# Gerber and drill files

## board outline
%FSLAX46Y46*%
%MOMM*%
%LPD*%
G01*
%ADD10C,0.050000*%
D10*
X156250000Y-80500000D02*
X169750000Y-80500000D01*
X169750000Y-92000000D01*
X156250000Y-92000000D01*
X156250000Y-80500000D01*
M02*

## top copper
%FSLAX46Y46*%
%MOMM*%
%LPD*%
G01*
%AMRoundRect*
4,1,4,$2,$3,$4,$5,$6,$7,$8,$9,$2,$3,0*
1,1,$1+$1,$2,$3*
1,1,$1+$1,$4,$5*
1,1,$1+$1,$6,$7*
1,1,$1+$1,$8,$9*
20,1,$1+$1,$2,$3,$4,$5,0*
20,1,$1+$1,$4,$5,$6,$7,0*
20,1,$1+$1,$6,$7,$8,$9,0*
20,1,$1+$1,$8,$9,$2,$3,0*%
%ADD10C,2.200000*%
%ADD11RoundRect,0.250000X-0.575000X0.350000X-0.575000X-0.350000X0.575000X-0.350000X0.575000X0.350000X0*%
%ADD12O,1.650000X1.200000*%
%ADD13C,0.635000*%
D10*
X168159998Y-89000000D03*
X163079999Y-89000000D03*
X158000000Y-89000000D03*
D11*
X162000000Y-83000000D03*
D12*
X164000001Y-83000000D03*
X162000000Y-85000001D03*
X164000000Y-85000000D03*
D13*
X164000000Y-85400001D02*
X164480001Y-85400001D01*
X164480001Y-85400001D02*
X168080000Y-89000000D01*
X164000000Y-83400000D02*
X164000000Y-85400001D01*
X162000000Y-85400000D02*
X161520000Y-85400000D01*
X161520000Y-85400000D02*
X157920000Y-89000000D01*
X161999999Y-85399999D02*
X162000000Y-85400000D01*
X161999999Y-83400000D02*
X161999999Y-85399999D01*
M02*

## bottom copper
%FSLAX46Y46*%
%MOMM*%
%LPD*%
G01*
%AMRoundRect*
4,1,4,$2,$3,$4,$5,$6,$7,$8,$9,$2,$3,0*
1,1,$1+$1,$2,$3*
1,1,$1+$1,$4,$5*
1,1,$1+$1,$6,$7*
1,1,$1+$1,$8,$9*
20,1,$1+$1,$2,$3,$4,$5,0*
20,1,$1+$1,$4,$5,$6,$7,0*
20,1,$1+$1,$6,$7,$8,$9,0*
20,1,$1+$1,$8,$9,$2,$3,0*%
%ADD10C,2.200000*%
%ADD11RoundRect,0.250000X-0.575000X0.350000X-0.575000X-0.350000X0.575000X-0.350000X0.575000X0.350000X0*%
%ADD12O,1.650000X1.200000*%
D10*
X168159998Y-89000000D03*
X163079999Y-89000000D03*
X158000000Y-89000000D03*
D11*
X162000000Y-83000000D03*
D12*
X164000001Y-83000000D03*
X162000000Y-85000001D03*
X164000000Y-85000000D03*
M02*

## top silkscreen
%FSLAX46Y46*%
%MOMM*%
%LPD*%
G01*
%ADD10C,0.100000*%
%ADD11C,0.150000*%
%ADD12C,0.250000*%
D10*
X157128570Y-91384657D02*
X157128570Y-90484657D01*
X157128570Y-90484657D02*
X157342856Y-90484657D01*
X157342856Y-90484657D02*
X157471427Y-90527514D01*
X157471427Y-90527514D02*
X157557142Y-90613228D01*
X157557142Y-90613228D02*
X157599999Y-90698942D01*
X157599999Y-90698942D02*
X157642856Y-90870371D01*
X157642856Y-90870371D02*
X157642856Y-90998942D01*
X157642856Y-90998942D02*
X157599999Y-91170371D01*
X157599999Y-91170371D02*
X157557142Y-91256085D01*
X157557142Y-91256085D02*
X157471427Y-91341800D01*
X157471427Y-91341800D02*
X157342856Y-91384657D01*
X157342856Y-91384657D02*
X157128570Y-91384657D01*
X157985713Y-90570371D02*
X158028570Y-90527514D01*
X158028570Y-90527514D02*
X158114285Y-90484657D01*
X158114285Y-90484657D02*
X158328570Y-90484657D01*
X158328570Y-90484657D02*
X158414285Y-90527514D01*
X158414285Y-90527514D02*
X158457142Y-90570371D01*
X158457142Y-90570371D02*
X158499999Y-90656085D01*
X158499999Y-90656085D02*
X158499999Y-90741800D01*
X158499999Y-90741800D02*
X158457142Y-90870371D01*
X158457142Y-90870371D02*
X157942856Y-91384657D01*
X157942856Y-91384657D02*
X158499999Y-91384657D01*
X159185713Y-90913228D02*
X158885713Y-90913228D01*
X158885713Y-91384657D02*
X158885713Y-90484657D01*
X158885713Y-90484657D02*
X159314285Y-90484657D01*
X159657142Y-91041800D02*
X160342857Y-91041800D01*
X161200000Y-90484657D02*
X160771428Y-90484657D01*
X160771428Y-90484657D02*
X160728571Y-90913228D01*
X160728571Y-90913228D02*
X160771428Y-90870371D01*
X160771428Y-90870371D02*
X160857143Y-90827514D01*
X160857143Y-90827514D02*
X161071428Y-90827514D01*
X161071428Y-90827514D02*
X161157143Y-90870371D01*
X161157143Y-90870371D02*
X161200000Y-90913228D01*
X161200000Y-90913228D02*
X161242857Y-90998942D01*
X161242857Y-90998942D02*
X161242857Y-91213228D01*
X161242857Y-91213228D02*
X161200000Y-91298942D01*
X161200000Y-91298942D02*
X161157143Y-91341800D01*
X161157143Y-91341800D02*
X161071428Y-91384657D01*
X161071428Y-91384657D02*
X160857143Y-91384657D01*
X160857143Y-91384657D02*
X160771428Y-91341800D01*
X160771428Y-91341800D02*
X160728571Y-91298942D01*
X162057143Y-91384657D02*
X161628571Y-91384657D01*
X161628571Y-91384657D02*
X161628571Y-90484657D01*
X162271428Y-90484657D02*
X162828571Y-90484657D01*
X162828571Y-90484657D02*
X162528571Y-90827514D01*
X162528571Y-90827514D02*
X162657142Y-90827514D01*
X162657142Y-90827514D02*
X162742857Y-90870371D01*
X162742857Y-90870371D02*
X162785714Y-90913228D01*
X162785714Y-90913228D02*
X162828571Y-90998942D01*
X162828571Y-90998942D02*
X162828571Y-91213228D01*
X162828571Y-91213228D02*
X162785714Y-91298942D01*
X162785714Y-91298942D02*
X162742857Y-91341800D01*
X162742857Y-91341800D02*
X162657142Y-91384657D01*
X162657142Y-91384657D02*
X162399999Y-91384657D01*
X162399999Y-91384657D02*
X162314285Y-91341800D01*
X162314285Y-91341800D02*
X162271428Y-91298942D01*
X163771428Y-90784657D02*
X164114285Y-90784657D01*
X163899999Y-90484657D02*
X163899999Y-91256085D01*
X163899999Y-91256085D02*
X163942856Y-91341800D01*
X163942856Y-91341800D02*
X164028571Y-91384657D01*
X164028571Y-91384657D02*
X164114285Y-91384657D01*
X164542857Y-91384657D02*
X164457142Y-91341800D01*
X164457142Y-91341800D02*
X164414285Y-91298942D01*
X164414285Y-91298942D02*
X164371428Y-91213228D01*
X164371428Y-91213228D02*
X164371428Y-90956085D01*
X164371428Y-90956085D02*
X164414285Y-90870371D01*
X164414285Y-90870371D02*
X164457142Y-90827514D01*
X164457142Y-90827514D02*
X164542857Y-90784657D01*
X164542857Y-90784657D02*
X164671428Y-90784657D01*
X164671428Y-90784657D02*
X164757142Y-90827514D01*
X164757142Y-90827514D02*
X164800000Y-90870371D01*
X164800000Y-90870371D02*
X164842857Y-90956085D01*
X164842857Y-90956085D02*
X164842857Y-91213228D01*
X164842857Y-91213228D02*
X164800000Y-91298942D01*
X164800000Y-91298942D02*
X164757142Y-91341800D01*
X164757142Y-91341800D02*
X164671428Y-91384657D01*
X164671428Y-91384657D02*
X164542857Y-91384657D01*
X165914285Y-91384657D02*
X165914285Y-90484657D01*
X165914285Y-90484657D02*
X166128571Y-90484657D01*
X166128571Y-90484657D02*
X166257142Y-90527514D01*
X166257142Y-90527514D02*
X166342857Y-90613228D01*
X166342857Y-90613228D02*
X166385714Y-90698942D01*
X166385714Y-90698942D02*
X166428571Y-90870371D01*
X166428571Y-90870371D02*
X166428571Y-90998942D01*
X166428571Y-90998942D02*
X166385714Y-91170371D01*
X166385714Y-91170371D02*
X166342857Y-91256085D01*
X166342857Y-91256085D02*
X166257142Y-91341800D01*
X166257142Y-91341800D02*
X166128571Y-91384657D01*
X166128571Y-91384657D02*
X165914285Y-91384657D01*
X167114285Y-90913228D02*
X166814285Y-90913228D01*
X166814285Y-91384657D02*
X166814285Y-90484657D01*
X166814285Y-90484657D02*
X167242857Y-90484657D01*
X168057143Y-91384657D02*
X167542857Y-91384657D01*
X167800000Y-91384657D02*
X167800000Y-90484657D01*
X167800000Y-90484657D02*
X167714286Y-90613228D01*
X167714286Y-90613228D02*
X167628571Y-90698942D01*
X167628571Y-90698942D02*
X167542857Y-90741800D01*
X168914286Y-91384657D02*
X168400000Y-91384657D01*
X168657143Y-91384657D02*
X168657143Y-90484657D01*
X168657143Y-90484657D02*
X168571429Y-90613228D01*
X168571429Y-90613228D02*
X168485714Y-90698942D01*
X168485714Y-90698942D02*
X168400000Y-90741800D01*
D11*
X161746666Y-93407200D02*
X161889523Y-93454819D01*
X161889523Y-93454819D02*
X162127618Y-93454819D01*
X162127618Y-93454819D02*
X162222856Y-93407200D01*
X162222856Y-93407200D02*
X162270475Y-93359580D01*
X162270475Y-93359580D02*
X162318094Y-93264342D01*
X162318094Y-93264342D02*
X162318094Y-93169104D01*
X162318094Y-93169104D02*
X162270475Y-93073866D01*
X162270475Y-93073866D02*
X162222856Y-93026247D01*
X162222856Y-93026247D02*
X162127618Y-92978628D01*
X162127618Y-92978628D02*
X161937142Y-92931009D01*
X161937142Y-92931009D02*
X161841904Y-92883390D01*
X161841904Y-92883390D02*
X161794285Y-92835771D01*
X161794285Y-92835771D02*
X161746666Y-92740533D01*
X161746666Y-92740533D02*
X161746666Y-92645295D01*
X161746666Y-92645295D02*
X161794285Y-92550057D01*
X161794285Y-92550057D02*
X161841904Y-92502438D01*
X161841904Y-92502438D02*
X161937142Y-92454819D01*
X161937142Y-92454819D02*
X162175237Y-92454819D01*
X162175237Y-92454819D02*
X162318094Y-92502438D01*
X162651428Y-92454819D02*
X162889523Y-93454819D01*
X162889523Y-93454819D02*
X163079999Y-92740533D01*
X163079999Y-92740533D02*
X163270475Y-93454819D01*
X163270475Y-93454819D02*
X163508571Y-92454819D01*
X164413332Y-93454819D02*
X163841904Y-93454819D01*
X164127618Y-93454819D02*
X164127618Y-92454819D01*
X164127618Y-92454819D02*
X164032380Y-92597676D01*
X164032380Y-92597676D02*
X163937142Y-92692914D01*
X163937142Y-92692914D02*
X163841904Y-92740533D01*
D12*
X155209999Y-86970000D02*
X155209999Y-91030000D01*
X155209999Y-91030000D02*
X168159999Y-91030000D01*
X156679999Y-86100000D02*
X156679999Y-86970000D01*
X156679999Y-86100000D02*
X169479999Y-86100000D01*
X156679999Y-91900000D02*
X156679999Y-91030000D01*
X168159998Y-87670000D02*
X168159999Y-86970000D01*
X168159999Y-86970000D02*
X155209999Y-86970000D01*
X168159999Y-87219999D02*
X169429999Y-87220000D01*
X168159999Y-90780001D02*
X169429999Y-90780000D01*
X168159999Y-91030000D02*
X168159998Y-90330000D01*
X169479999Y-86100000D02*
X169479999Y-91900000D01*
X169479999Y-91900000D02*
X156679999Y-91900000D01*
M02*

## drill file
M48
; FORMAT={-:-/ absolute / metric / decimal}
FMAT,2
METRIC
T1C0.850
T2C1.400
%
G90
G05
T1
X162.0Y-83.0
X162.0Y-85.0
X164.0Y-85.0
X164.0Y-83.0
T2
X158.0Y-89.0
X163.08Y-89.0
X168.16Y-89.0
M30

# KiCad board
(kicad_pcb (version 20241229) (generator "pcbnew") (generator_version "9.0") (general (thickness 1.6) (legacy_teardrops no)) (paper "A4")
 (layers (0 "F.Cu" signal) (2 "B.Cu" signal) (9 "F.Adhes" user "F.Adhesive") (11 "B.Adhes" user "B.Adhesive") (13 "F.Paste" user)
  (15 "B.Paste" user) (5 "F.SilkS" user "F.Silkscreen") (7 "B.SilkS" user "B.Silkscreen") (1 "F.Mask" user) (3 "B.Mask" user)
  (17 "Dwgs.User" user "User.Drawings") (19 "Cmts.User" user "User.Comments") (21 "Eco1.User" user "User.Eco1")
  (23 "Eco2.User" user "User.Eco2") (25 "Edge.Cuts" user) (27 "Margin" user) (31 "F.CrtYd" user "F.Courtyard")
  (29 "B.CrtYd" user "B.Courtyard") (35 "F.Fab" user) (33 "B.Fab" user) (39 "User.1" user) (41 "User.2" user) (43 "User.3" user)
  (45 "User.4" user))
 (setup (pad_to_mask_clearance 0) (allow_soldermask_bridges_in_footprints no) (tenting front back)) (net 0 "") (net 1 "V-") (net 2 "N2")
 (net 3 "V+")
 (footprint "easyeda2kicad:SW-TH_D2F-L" (layer "F.Cu") (at 163.079999 89 180)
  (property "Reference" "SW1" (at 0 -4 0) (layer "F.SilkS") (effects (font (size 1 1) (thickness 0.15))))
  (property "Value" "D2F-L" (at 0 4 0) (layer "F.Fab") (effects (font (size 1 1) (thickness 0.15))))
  (fp_line (start 7.87 2.03) (end 7.87 -2.03) (stroke (width 0.25) (type solid)) (layer "F.SilkS"))
  (fp_line (start 7.87 -2.03) (end -5.08 -2.03) (stroke (width 0.25) (type solid)) (layer "F.SilkS"))
  (fp_line (start 6.4 2.9) (end 6.4 2.03) (stroke (width 0.25) (type solid)) (layer "F.SilkS"))
  (fp_line (start 6.4 2.9) (end -6.4 2.9) (stroke (width 0.25) (type solid)) (layer "F.SilkS"))
  (fp_line (start 6.4 -2.9) (end 6.4 -2.03) (stroke (width 0.25) (type solid)) (layer "F.SilkS"))
  (fp_line (start -5.079999 1.33) (end -5.08 2.03) (stroke (width 0.25) (type solid)) (layer "F.SilkS"))
  (fp_line (start -5.08 2.03) (end 7.87 2.03) (stroke (width 0.25) (type solid)) (layer "F.SilkS"))
  (fp_line (start -5.08 1.780001) (end -6.35 1.78) (stroke (width 0.25) (type solid)) (layer "F.SilkS"))
  (fp_line (start -5.08 -1.780001) (end -6.35 -1.78) (stroke (width 0.25) (type solid)) (layer "F.SilkS"))
  (fp_line (start -5.08 -2.03) (end -5.079999 -1.33) (stroke (width 0.25) (type solid)) (layer "F.SilkS"))
  (fp_line (start -6.4 2.9) (end -6.4 -2.9) (stroke (width 0.25) (type solid)) (layer "F.SilkS"))
  (fp_line (start -6.4 -2.9) (end 6.4 -2.9) (stroke (width 0.25) (type solid)) (layer "F.SilkS"))
  (pad "1" thru_hole circle (at -5.079999 0 180) (size 2.2 2.2) (drill 1.399997) (layers "*.Cu" "*.Mask") (remove_unused_layers no)
   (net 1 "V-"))
  (pad "2" thru_hole circle (at 0 0 180) (size 2.2 2.2) (drill 1.399997) (layers "*.Cu" "*.Mask") (remove_unused_layers no) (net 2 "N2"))
  (pad "3" thru_hole circle (at 5.079999 0 180) (size 2.2 2.2) (drill 1.399997) (layers "*.Cu" "*.Mask") (remove_unused_layers no)
   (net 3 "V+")))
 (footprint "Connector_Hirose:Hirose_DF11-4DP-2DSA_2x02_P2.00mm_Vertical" (layer "B.Cu") (at 162 83 -90)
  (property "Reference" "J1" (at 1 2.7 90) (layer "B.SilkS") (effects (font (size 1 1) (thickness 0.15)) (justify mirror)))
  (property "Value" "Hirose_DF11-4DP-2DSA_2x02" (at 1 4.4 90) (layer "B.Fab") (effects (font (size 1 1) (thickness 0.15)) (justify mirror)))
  (pad "1" thru_hole roundrect (at 0 0 270) (size 1.2 1.65) (drill 0.85) (layers "*.Cu" "*.Mask") (remove_unused_layers no)
   (roundrect_rratio 0.208333) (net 1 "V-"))
  (pad "2" thru_hole oval (at 0 -2.000001 270) (size 1.2 1.65) (drill 0.85) (layers "*.Cu" "*.Mask") (remove_unused_layers no) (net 3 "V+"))
  (pad "3" thru_hole oval (at 2.000001 0 270) (size 1.2 1.65) (drill 0.85) (layers "*.Cu" "*.Mask") (remove_unused_layers no) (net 1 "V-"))
  (pad "4" thru_hole oval (at 2 -2 270) (size 1.2 1.65) (drill 0.85) (layers "*.Cu" "*.Mask") (remove_unused_layers no) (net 3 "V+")))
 (gr_rect (start 156.25 80.5) (end 169.75 92) (stroke (width 0.05) (type default)) (fill no) (layer "Edge.Cuts"))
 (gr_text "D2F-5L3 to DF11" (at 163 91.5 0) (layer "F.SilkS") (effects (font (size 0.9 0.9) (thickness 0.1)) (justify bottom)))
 (segment (start 164 85.400001) (end 164.480001 85.400001) (width 0.635) (layer "F.Cu") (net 1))
 (segment (start 164.480001 85.400001) (end 168.08 89) (width 0.635) (layer "F.Cu") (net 1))
 (segment (start 164 83.4) (end 164 85.400001) (width 0.635) (layer "F.Cu") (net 1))
 (segment (start 162 85.4) (end 161.52 85.4) (width 0.635) (layer "F.Cu") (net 3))
 (segment (start 161.52 85.4) (end 157.92 89) (width 0.635) (layer "F.Cu") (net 3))
 (segment (start 161.999999 85.399999) (end 162 85.4) (width 0.635) (layer "F.Cu") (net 3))
 (segment (start 161.999999 83.4) (end 161.999999 85.399999) (width 0.635) (layer "F.Cu") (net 3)))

